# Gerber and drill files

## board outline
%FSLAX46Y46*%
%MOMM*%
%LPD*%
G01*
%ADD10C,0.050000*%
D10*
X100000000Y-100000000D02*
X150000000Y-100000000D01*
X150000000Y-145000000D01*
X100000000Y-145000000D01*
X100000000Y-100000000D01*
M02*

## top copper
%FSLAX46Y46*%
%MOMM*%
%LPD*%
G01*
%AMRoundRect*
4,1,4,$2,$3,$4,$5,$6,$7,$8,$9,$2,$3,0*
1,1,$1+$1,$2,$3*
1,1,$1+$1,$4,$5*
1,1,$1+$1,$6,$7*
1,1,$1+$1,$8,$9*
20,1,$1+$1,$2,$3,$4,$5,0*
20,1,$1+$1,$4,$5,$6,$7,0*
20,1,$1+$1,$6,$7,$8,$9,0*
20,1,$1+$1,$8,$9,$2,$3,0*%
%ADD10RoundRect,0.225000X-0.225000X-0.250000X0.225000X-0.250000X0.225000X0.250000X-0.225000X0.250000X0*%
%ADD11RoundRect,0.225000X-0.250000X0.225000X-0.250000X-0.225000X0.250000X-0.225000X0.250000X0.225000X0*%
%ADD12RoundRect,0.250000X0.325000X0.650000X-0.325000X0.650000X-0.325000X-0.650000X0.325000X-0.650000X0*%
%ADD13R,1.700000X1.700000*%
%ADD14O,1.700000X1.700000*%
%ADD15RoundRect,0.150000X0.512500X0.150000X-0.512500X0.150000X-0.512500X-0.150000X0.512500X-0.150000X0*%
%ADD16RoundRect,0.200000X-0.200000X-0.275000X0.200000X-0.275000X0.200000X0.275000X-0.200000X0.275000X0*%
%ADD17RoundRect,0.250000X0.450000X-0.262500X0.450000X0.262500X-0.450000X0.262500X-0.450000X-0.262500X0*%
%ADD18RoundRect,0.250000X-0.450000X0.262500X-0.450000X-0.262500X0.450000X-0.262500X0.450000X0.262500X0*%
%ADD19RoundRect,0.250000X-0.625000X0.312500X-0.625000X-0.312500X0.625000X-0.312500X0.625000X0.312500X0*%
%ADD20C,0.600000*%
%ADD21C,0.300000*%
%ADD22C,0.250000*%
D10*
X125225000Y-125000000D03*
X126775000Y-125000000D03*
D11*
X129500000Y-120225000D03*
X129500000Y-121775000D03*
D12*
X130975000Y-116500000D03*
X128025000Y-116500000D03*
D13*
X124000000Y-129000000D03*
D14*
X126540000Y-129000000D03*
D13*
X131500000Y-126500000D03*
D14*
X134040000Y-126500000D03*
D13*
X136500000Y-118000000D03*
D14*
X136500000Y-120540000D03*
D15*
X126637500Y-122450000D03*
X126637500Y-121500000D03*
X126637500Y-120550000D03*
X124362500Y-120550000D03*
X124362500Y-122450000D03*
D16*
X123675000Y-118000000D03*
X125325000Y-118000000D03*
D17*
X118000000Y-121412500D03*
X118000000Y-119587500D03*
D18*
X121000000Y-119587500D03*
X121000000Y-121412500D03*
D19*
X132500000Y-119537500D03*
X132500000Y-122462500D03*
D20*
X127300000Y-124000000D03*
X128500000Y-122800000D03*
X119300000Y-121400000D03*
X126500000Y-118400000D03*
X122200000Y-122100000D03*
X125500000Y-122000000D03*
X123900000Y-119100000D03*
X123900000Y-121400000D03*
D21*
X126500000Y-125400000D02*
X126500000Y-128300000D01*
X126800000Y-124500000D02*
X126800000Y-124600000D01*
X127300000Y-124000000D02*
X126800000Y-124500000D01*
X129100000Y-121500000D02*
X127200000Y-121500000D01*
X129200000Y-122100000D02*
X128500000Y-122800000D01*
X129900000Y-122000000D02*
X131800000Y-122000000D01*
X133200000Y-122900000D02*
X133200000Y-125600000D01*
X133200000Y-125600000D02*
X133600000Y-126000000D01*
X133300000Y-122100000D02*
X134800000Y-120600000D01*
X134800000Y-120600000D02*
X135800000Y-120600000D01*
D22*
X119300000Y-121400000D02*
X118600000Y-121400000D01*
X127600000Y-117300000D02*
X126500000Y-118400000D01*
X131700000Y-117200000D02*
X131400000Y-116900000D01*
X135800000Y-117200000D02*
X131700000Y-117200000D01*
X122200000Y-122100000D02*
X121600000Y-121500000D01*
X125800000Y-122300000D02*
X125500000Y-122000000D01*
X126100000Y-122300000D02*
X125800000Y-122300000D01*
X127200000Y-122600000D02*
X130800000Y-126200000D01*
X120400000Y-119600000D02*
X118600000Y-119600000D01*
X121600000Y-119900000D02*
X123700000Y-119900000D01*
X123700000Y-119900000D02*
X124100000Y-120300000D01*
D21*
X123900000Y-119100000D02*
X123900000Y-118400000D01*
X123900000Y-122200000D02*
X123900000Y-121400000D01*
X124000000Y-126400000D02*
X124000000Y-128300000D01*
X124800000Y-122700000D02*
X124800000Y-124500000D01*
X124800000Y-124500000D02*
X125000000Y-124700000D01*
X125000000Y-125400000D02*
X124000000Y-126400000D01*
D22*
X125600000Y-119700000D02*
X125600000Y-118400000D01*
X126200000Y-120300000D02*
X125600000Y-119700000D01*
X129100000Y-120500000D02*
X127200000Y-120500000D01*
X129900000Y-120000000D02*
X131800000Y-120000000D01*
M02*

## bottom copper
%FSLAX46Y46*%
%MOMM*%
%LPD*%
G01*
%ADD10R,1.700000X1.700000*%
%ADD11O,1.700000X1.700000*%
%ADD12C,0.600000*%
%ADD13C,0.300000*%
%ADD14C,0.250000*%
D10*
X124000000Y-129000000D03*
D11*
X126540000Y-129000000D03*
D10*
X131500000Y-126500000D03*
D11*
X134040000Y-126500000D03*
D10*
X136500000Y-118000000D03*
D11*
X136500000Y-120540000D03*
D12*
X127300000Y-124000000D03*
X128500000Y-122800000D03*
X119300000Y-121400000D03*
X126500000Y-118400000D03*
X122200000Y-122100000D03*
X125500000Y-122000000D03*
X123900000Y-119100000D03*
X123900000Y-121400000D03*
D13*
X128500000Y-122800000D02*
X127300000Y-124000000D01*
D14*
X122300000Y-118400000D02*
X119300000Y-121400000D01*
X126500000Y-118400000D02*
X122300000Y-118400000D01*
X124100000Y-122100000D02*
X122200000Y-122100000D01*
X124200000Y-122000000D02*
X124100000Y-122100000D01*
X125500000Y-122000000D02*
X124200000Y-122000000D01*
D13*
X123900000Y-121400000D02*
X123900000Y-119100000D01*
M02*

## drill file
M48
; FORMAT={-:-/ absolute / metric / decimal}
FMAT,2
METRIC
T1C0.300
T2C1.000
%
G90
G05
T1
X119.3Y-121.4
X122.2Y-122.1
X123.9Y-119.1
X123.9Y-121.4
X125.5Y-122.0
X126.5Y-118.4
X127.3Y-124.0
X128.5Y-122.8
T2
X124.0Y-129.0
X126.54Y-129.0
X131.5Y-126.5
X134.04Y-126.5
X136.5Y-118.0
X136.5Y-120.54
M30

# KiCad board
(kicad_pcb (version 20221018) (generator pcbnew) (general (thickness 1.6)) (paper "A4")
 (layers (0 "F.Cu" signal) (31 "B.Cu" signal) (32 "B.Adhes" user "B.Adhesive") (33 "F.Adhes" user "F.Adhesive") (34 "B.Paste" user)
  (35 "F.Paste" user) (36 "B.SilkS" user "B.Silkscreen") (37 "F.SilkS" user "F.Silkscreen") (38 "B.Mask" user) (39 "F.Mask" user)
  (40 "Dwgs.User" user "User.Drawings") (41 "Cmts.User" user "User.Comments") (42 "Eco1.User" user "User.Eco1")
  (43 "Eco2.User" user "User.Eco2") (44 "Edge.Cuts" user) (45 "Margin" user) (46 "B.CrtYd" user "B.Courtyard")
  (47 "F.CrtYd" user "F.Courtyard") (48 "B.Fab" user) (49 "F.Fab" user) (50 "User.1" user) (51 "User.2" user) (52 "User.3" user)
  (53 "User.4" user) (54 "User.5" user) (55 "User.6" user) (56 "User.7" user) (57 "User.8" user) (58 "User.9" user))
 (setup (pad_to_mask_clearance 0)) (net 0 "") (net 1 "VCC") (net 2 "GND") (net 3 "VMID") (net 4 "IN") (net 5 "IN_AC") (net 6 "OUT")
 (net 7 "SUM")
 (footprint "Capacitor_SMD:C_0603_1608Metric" (layer "F.Cu") (at 126 125)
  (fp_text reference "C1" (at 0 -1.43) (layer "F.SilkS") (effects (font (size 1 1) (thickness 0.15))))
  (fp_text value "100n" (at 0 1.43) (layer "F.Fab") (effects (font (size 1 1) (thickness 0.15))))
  (pad "1" smd roundrect (at -0.775 0) (size 0.9 0.95) (layers "F.Cu" "F.Paste" "F.Mask") (roundrect_rratio 0.25) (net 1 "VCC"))
  (pad "2" smd roundrect (at 0.775 0) (size 0.9 0.95) (layers "F.Cu" "F.Paste" "F.Mask") (roundrect_rratio 0.25) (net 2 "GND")))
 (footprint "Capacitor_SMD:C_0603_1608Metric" (layer "F.Cu") (at 129.5 121 -90)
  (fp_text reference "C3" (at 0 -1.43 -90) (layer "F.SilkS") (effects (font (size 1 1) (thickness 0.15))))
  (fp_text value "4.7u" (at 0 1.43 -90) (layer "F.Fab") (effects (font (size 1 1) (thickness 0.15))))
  (pad "1" smd roundrect (at -0.775 0 270) (size 0.9 0.95) (layers "F.Cu" "F.Paste" "F.Mask") (roundrect_rratio 0.25) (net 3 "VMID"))
  (pad "2" smd roundrect (at 0.775 0 270) (size 0.9 0.95) (layers "F.Cu" "F.Paste" "F.Mask") (roundrect_rratio 0.25) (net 2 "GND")))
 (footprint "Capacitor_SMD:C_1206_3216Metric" (layer "F.Cu") (at 129.5 116.5 180)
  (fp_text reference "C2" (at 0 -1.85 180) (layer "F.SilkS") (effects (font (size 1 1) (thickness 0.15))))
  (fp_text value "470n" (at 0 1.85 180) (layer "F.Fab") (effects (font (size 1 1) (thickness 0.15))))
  (pad "1" smd roundrect (at -1.475 0 180) (size 1.15 1.8) (layers "F.Cu" "F.Paste" "F.Mask") (roundrect_rratio 0.217391) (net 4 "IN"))
  (pad "2" smd roundrect (at 1.475 0 180) (size 1.15 1.8) (layers "F.Cu" "F.Paste" "F.Mask") (roundrect_rratio 0.217391) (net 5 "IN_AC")))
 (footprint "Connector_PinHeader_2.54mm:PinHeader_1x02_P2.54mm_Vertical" (layer "F.Cu") (at 124 129 90)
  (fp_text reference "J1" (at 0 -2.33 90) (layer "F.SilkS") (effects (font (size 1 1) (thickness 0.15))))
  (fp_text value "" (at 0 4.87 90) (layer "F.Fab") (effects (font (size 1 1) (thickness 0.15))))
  (pad "1" thru_hole rect (at 0 0 90) (size 1.7 1.7) (drill 1) (layers "*.Cu" "*.Mask") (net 1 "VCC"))
  (pad "2" thru_hole oval (at 0 2.54 90) (size 1.7 1.7) (drill 1) (layers "*.Cu" "*.Mask") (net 2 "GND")))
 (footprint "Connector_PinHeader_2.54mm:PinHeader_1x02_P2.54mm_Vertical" (layer "F.Cu") (at 131.5 126.5 90)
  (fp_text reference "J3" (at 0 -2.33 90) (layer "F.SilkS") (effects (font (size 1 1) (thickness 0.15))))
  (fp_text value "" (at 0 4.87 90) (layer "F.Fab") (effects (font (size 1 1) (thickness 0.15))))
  (pad "1" thru_hole rect (at 0 0 90) (size 1.7 1.7) (drill 1) (layers "*.Cu" "*.Mask") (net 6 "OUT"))
  (pad "2" thru_hole oval (at 0 2.54 90) (size 1.7 1.7) (drill 1) (layers "*.Cu" "*.Mask") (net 2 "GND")))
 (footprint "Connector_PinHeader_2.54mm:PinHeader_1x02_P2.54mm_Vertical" (layer "F.Cu") (at 136.5 118)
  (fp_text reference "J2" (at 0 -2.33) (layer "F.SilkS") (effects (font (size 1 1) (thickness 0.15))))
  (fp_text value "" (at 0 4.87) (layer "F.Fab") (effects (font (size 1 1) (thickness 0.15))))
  (pad "1" thru_hole rect (at 0 0) (size 1.7 1.7) (drill 1) (layers "*.Cu" "*.Mask") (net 4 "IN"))
  (pad "2" thru_hole oval (at 0 2.54) (size 1.7 1.7) (drill 1) (layers "*.Cu" "*.Mask") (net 2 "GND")))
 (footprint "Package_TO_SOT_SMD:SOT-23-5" (layer "F.Cu") (at 125.5 121.5 180)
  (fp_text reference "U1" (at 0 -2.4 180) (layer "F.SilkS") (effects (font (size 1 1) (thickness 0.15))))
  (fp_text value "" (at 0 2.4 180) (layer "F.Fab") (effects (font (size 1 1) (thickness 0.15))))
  (pad "1" smd roundrect (at -1.1375 -0.95 180) (size 1.325 0.6) (layers "F.Cu" "F.Paste" "F.Mask") (roundrect_rratio 0.25) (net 6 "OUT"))
  (pad "2" smd roundrect (at -1.1375 0 180) (size 1.325 0.6) (layers "F.Cu" "F.Paste" "F.Mask") (roundrect_rratio 0.25) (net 2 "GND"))
  (pad "3" smd roundrect (at -1.1375 0.95 180) (size 1.325 0.6) (layers "F.Cu" "F.Paste" "F.Mask") (roundrect_rratio 0.25) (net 3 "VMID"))
  (pad "4" smd roundrect (at 1.1375 0.95 180) (size 1.325 0.6) (layers "F.Cu" "F.Paste" "F.Mask") (roundrect_rratio 0.25) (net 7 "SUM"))
  (pad "5" smd roundrect (at 1.1375 -0.95 180) (size 1.325 0.6) (layers "F.Cu" "F.Paste" "F.Mask") (roundrect_rratio 0.25) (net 1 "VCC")))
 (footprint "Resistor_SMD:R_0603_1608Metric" (layer "F.Cu") (at 124.5 118)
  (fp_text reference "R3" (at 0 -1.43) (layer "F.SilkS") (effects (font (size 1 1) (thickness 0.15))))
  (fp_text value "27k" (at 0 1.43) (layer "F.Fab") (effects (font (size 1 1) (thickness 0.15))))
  (pad "1" smd roundrect (at -0.825 0) (size 0.8 0.95) (layers "F.Cu" "F.Paste" "F.Mask") (roundrect_rratio 0.25) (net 1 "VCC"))
  (pad "2" smd roundrect (at 0.825 0) (size 0.8 0.95) (layers "F.Cu" "F.Paste" "F.Mask") (roundrect_rratio 0.25) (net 3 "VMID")))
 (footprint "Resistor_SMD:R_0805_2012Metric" (layer "F.Cu") (at 118 120.5 90)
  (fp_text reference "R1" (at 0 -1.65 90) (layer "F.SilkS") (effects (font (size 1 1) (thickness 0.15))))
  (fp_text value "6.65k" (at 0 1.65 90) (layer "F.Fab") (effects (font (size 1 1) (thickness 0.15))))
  (pad "1" smd roundrect (at -0.9125 0 90) (size 1.025 1.4) (layers "F.Cu" "F.Paste" "F.Mask") (roundrect_rratio 0.243902) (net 5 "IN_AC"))
  (pad "2" smd roundrect (at 0.9125 0 90) (size 1.025 1.4) (layers "F.Cu" "F.Paste" "F.Mask") (roundrect_rratio 0.243902) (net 7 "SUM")))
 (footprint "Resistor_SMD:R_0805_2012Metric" (layer "F.Cu") (at 121 120.5 -90)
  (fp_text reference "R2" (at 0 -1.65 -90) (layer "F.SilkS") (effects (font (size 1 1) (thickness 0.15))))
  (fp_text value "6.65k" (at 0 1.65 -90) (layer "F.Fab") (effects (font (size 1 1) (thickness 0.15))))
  (pad "1" smd roundrect (at -0.9125 0 270) (size 1.025 1.4) (layers "F.Cu" "F.Paste" "F.Mask") (roundrect_rratio 0.243902) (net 7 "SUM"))
  (pad "2" smd roundrect (at 0.9125 0 270) (size 1.025 1.4) (layers "F.Cu" "F.Paste" "F.Mask") (roundrect_rratio 0.243902) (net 6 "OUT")))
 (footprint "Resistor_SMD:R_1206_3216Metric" (layer "F.Cu") (at 132.5 121 -90)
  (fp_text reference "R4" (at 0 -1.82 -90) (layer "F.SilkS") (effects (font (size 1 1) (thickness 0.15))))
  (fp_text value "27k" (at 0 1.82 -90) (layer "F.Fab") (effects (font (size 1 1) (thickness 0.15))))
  (pad "1" smd roundrect (at -1.4625 0 270) (size 1.125 1.75) (layers "F.Cu" "F.Paste" "F.Mask") (roundrect_rratio 0.222222) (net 3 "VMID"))
  (pad "2" smd roundrect (at 1.4625 0 270) (size 1.125 1.75) (layers "F.Cu" "F.Paste" "F.Mask") (roundrect_rratio 0.222222) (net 2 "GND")))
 (gr_rect (start 100 100) (end 150 145) (stroke (width 0.05) (type default)) (fill none) (layer "Edge.Cuts"))
 (segment (start 126.5 125.4) (end 126.5 128.3) (width 0.3) (layer "F.Cu") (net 2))
 (segment (start 126.8 124.5) (end 126.8 124.6) (width 0.3) (layer "F.Cu") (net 2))
 (segment (start 127.3 124) (end 126.8 124.5) (width 0.3) (layer "F.Cu") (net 2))
 (segment (start 129.1 121.5) (end 127.2 121.5) (width 0.3) (layer "F.Cu") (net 2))
 (segment (start 129.2 122.1) (end 128.5 122.8) (width 0.3) (layer "F.Cu") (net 2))
 (segment (start 129.9 122) (end 131.8 122) (width 0.3) (layer "F.Cu") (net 2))
 (segment (start 133.2 122.9) (end 133.2 125.6) (width 0.3) (layer "F.Cu") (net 2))
 (segment (start 133.2 125.6) (end 133.6 126) (width 0.3) (layer "F.Cu") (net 2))
 (segment (start 133.3 122.1) (end 134.8 120.6) (width 0.3) (layer "F.Cu") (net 2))
 (segment (start 134.8 120.6) (end 135.8 120.6) (width 0.3) (layer "F.Cu") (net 2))
 (via (at 127.3 124) (size 0.6) (drill 0.3) (layers "F.Cu" "B.Cu") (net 2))
 (via (at 128.5 122.8) (size 0.6) (drill 0.3) (layers "F.Cu" "B.Cu") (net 2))
 (segment (start 119.3 121.4) (end 118.6 121.4) (width 0.25) (layer "F.Cu") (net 5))
 (segment (start 127.6 117.3) (end 126.5 118.4) (width 0.25) (layer "F.Cu") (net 5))
 (segment (start 128.5 122.8) (end 127.3 124) (width 0.3) (layer "B.Cu") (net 2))
 (segment (start 131.7 117.2) (end 131.4 116.9) (width 0.25) (layer "F.Cu") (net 4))
 (segment (start 135.8 117.2) (end 131.7 117.2) (width 0.25) (layer "F.Cu") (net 4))
 (via (at 119.3 121.4) (size 0.6) (drill 0.3) (layers "F.Cu" "B.Cu") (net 5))
 (via (at 126.5 118.4) (size 0.6) (drill 0.3) (layers "F.Cu" "B.Cu") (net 5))
 (segment (start 122.2 122.1) (end 121.6 121.5) (width 0.25) (layer "F.Cu") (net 6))
 (segment (start 122.3 118.4) (end 119.3 121.4) (width 0.25) (layer "B.Cu") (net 5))
 (segment (start 125.8 122.3) (end 125.5 122) (width 0.25) (layer "F.Cu") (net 6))
 (segment (start 126.1 122.3) (end 125.8 122.3) (width 0.25) (layer "F.Cu") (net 6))
 (segment (start 126.5 118.4) (end 122.3 118.4) (width 0.25) (layer "B.Cu") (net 5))
 (segment (start 127.2 122.6) (end 130.8 126.2) (width 0.25) (layer "F.Cu") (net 6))
 (via (at 122.2 122.1) (size 0.6) (drill 0.3) (layers "F.Cu" "B.Cu") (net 6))
 (via (at 125.5 122) (size 0.6) (drill 0.3) (layers "F.Cu" "B.Cu") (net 6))
 (segment (start 120.4 119.6) (end 118.6 119.6) (width 0.25) (layer "F.Cu") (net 7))
 (segment (start 121.6 119.9) (end 123.7 119.9) (width 0.25) (layer "F.Cu") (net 7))
 (segment (start 123.7 119.9) (end 124.1 120.3) (width 0.25) (layer "F.Cu") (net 7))
 (segment (start 123.9 119.1) (end 123.9 118.4) (width 0.3) (layer "F.Cu") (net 1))
 (segment (start 123.9 122.2) (end 123.9 121.4) (width 0.3) (layer "F.Cu") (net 1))
 (segment (start 124 126.4) (end 124 128.3) (width 0.3) (layer "F.Cu") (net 1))
 (segment (start 124.1 122.1) (end 122.2 122.1) (width 0.25) (layer "B.Cu") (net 6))
 (segment (start 124.2 122) (end 124.1 122.1) (width 0.25) (layer "B.Cu") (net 6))
 (segment (start 124.8 122.7) (end 124.8 124.5) (width 0.3) (layer "F.Cu") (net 1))
 (segment (start 124.8 124.5) (end 125 124.7) (width 0.3) (layer "F.Cu") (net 1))
 (segment (start 125 125.4) (end 124 126.4) (width 0.3) (layer "F.Cu") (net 1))
 (segment (start 125.5 122) (end 124.2 122) (width 0.25) (layer "B.Cu") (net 6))
 (via (at 123.9 119.1) (size 0.6) (drill 0.3) (layers "F.Cu" "B.Cu") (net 1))
 (via (at 123.9 121.4) (size 0.6) (drill 0.3) (layers "F.Cu" "B.Cu") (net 1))
 (segment (start 123.9 121.4) (end 123.9 119.1) (width 0.3) (layer "B.Cu") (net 1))
 (segment (start 125.6 119.7) (end 125.6 118.4) (width 0.25) (layer "F.Cu") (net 3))
 (segment (start 126.2 120.3) (end 125.6 119.7) (width 0.25) (layer "F.Cu") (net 3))
 (segment (start 129.1 120.5) (end 127.2 120.5) (width 0.25) (layer "F.Cu") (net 3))
 (segment (start 129.9 120) (end 131.8 120) (width 0.25) (layer "F.Cu") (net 3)))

